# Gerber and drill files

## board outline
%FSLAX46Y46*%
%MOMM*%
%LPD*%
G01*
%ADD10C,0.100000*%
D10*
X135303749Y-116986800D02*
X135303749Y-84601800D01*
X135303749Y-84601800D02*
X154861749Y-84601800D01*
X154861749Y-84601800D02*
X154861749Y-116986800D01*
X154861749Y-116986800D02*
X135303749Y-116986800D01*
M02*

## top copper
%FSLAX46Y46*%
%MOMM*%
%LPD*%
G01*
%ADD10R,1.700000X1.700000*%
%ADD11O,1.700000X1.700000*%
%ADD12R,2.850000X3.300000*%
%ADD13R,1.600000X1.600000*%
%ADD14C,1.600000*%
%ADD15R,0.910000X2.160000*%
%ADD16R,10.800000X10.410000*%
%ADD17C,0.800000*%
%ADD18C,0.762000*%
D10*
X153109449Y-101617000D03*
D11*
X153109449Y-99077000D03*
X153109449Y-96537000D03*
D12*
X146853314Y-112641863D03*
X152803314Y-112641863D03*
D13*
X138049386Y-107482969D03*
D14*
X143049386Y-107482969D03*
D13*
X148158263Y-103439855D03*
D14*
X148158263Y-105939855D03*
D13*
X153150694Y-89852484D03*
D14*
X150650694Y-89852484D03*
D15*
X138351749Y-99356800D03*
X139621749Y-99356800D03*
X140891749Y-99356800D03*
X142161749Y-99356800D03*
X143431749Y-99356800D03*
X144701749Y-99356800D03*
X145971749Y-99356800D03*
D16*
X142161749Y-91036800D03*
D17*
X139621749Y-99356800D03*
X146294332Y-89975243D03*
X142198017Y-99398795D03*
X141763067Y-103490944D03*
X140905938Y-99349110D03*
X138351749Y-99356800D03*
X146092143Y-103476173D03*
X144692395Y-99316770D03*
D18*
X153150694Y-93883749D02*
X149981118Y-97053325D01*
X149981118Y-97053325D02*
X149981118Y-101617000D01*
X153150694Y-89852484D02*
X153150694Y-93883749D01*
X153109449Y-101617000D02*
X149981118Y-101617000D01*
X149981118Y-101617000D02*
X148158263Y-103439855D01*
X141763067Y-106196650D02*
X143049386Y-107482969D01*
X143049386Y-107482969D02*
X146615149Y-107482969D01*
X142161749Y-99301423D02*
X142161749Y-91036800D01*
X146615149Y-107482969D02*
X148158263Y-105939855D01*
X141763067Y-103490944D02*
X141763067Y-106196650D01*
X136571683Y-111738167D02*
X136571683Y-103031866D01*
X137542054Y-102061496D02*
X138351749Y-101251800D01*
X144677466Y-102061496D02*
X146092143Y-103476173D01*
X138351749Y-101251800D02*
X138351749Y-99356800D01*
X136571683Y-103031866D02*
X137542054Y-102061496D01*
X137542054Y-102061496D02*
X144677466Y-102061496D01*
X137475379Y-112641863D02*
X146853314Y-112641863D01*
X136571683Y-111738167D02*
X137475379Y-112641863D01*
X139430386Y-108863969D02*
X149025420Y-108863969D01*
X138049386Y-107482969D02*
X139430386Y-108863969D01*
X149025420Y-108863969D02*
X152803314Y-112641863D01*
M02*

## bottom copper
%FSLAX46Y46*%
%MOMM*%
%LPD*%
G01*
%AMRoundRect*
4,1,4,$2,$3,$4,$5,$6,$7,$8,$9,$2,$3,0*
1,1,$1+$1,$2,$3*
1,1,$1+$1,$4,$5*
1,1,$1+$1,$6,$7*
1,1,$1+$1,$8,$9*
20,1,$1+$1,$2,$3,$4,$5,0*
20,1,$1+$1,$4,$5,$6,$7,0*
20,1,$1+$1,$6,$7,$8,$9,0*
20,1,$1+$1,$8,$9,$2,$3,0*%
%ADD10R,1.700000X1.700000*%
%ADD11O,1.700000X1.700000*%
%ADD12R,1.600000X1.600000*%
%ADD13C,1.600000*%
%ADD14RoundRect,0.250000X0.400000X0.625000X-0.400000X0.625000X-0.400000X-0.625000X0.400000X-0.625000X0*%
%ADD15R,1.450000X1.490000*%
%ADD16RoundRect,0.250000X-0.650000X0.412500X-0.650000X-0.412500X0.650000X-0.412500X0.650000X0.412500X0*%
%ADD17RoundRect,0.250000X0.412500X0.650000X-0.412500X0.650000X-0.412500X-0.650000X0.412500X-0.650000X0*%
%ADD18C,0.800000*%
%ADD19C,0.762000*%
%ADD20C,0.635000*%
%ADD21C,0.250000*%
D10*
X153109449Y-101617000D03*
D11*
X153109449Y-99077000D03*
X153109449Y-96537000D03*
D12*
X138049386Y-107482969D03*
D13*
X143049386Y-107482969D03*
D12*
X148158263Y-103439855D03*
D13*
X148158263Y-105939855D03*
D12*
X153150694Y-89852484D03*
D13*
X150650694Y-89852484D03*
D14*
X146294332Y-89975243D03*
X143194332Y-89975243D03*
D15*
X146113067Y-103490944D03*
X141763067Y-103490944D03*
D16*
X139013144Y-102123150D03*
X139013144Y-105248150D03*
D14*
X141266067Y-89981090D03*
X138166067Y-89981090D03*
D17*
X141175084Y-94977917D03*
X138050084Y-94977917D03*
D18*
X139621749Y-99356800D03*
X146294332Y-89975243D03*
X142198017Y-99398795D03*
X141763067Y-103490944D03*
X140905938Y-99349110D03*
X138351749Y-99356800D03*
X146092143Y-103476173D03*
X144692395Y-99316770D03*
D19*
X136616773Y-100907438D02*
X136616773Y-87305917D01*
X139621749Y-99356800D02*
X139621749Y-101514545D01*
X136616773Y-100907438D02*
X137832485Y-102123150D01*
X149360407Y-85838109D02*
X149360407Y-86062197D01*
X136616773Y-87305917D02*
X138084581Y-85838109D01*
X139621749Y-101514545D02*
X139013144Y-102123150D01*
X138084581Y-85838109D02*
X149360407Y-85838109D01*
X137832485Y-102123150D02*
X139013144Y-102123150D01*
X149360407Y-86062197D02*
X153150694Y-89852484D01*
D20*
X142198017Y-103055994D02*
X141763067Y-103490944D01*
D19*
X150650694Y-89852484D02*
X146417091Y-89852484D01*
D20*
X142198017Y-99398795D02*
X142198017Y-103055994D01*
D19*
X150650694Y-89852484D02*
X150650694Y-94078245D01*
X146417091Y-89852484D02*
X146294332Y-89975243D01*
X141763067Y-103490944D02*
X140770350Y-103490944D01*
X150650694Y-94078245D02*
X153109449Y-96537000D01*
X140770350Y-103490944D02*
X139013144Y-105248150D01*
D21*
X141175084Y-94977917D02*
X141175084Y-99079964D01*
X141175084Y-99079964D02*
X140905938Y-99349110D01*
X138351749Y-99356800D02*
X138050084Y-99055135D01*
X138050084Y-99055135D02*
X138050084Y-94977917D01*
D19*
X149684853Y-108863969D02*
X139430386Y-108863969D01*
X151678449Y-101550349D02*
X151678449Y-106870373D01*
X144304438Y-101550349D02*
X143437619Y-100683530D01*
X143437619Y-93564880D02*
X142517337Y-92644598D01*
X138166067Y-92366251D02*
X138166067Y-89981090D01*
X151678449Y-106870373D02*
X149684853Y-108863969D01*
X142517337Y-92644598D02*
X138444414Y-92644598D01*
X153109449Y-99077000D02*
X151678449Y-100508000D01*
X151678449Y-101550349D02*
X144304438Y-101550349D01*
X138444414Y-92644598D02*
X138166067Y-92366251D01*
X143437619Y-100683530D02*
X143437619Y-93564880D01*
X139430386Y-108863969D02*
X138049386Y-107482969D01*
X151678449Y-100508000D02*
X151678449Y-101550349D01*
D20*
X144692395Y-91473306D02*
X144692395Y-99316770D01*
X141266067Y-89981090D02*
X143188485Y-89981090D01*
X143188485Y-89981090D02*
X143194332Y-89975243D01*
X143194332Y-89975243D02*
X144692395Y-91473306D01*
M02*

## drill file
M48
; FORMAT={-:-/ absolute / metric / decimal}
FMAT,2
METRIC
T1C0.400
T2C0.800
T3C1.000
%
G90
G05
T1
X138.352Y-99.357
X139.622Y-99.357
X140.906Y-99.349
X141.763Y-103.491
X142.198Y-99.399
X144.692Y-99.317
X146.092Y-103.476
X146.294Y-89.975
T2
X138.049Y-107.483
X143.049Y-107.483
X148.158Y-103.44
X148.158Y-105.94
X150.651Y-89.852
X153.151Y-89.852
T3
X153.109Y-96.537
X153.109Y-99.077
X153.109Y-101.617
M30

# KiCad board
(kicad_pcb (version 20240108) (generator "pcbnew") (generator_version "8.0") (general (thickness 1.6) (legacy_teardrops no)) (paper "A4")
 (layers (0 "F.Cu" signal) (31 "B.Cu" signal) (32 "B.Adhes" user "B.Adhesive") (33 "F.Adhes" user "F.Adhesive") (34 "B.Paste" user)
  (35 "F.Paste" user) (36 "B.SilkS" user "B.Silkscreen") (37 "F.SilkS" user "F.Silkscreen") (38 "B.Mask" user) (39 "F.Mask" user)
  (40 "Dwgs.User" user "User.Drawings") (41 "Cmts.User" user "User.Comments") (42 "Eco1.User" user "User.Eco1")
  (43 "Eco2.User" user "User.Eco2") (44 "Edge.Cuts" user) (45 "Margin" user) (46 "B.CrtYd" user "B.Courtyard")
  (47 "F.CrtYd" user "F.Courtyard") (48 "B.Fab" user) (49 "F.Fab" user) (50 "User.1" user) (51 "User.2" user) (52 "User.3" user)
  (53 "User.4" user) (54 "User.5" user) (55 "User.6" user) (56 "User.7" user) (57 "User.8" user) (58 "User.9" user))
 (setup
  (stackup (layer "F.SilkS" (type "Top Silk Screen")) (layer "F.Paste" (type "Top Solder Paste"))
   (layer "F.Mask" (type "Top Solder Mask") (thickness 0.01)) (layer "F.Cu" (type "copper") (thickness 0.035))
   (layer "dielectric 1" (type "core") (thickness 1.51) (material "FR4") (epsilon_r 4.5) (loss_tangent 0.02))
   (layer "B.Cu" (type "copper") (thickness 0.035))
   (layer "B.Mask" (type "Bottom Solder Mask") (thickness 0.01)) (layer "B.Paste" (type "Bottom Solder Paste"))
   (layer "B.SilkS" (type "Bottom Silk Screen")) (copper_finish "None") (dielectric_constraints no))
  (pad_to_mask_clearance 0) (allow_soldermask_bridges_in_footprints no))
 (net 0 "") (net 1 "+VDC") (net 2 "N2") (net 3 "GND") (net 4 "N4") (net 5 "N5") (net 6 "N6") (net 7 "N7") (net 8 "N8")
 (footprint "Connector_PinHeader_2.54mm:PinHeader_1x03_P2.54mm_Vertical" (layer "F.Cu") (at 153.109449 101.617 180)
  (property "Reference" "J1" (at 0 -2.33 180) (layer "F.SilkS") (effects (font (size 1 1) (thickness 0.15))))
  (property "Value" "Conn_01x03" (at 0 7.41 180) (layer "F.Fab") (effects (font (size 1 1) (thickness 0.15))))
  (pad "1" thru_hole rect (at 0 0 180) (size 1.7 1.7) (drill 1) (layers "*.Cu" "*.Mask") (remove_unused_layers no) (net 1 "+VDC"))
  (pad "2" thru_hole oval (at 0 2.54 180) (size 1.7 1.7) (drill 1) (layers "*.Cu" "*.Mask") (remove_unused_layers no) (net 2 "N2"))
  (pad "3" thru_hole oval (at 0 5.08 180) (size 1.7 1.7) (drill 1) (layers "*.Cu" "*.Mask") (remove_unused_layers no) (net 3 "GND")))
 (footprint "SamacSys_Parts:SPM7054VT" (layer "F.Cu") (at 149.828314 112.641863)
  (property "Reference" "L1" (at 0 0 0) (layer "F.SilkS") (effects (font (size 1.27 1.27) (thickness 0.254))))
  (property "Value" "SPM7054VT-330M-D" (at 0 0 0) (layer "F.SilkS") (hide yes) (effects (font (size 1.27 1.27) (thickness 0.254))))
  (pad "1" smd rect (at -2.975 0) (size 2.85 3.3) (layers "F.Cu" "F.Paste" "F.Mask") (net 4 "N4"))
  (pad "2" smd rect (at 2.975 0) (size 2.85 3.3) (layers "F.Cu" "F.Paste" "F.Mask") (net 2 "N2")))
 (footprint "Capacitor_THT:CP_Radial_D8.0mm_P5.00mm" (layer "F.Cu") (at 138.049386 107.482969)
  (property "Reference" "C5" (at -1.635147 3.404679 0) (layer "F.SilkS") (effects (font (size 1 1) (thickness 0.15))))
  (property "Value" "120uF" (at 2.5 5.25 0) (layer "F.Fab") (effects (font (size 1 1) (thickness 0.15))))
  (pad "1" thru_hole rect (at 0 0) (size 1.6 1.6) (drill 0.8) (layers "*.Cu" "*.Mask") (remove_unused_layers no) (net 2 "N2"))
  (pad "2" thru_hole circle (at 5 0) (size 1.6 1.6) (drill 0.8) (layers "*.Cu" "*.Mask") (remove_unused_layers no) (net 3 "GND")))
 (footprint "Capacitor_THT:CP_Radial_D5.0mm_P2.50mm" (layer "F.Cu") (at 148.158263 103.439855 -90)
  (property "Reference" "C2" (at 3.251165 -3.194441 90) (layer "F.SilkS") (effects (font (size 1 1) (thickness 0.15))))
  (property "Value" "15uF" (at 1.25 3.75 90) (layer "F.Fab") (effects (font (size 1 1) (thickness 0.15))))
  (pad "1" thru_hole rect (at 0 0 270) (size 1.6 1.6) (drill 0.8) (layers "*.Cu" "*.Mask") (remove_unused_layers no) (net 1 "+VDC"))
  (pad "2" thru_hole circle (at 2.5 0 270) (size 1.6 1.6) (drill 0.8) (layers "*.Cu" "*.Mask") (remove_unused_layers no) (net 3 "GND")))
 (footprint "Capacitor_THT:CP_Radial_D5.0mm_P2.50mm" (layer "F.Cu") (at 153.150694 89.852484 180)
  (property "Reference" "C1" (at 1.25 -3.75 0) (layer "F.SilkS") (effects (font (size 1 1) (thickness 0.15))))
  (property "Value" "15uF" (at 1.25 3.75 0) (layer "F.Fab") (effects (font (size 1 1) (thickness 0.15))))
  (pad "1" thru_hole rect (at 0 0 180) (size 1.6 1.6) (drill 0.8) (layers "*.Cu" "*.Mask") (remove_unused_layers no) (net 1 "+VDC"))
  (pad "2" thru_hole circle (at 2.5 0 180) (size 1.6 1.6) (drill 0.8) (layers "*.Cu" "*.Mask") (remove_unused_layers no) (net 3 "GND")))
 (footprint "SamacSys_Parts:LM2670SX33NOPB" (layer "F.Cu") (at 142.161749 91.5868 -90)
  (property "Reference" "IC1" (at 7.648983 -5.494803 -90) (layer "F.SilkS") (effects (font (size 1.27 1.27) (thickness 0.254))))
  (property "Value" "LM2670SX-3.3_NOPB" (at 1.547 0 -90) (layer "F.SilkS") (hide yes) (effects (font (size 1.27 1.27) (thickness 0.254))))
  (pad "1" smd rect (at 7.77 3.81) (size 0.91 2.16) (layers "F.Cu" "F.Paste" "F.Mask") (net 4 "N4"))
  (pad "2" smd rect (at 7.77 2.54) (size 0.91 2.16) (layers "F.Cu" "F.Paste" "F.Mask") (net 1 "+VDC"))
  (pad "3" smd rect (at 7.77 1.27) (size 0.91 2.16) (layers "F.Cu" "F.Paste" "F.Mask") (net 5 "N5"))
  (pad "4" smd rect (at 7.77 0) (size 0.91 2.16) (layers "F.Cu" "F.Paste" "F.Mask") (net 3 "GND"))
  (pad "5" smd rect (at 7.77 -1.27) (size 0.91 2.16) (layers "F.Cu" "F.Paste" "F.Mask") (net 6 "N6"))
  (pad "6" smd rect (at 7.77 -2.54) (size 0.91 2.16) (layers "F.Cu" "F.Paste" "F.Mask") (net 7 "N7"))
  (pad "7" smd rect (at 7.77 -3.81) (size 0.91 2.16) (layers "F.Cu" "F.Paste" "F.Mask") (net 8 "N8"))
  (pad "8" smd rect (at -0.55 0 270) (size 10.41 10.8) (layers "F.Cu" "F.Paste" "F.Mask") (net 3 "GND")))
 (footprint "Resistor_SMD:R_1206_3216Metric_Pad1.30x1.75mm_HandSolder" (layer "B.Cu") (at 144.744332 89.975243 180)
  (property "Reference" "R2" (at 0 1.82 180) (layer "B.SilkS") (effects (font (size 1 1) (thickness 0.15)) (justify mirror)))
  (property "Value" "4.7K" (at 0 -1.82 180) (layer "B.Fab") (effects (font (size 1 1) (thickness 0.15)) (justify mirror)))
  (pad "1" smd roundrect (at -1.55 0 180) (size 1.3 1.75) (layers "B.Cu" "B.Paste" "B.Mask") (roundrect_rratio 0.192308) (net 3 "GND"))
  (pad "2" smd roundrect (at 1.55 0 180) (size 1.3 1.75) (layers "B.Cu" "B.Paste" "B.Mask") (roundrect_rratio 0.192308) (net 7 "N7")))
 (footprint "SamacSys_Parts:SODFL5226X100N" (layer "B.Cu") (at 143.938067 103.490944 180)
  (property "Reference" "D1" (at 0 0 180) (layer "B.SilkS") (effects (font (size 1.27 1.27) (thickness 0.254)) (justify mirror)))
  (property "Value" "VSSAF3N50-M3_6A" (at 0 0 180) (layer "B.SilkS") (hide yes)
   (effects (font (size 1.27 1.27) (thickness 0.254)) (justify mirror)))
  (pad "1" smd rect (at -2.175 0 180) (size 1.45 1.49) (layers "B.Cu" "B.Paste" "B.Mask") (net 4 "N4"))
  (pad "2" smd rect (at 2.175 0 180) (size 1.45 1.49) (layers "B.Cu" "B.Paste" "B.Mask") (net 3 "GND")))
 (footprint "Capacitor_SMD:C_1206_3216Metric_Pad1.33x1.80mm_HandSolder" (layer "B.Cu") (at 139.013144 103.68565 -90)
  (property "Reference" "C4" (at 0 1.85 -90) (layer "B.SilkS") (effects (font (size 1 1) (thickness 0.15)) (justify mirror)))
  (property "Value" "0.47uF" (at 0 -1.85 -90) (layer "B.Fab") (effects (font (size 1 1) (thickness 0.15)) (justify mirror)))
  (pad "1" smd roundrect (at -1.5625 0 270) (size 1.325 1.8) (layers "B.Cu" "B.Paste" "B.Mask") (roundrect_rratio 0.188679) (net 1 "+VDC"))
  (pad "2" smd roundrect (at 1.5625 0 270) (size 1.325 1.8) (layers "B.Cu" "B.Paste" "B.Mask") (roundrect_rratio 0.188679) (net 3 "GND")))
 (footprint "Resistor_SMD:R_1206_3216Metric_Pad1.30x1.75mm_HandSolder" (layer "B.Cu") (at 139.716067 89.98109 180)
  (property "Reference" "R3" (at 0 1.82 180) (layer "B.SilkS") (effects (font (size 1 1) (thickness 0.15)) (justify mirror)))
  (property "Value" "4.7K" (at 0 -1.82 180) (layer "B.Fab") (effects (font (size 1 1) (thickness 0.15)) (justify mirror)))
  (pad "1" smd roundrect (at -1.55 0 180) (size 1.3 1.75) (layers "B.Cu" "B.Paste" "B.Mask") (roundrect_rratio 0.192308) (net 7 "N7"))
  (pad "2" smd roundrect (at 1.55 0 180) (size 1.3 1.75) (layers "B.Cu" "B.Paste" "B.Mask") (roundrect_rratio 0.192308) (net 2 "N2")))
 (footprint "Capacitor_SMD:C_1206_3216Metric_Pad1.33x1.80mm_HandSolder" (layer "B.Cu") (at 139.612584 94.977917 180)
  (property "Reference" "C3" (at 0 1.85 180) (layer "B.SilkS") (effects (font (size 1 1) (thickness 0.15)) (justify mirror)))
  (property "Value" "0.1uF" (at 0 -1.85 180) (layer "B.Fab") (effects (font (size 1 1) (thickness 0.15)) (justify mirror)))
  (pad "1" smd roundrect (at -1.5625 0 180) (size 1.325 1.8) (layers "B.Cu" "B.Paste" "B.Mask") (roundrect_rratio 0.188679) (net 5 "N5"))
  (pad "2" smd roundrect (at 1.5625 0 180) (size 1.325 1.8) (layers "B.Cu" "B.Paste" "B.Mask") (roundrect_rratio 0.188679) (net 4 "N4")))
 (gr_line (start 135.303749 116.9868) (end 135.303749 84.6018) (stroke (width 0.1) (type solid)) (layer "Edge.Cuts"))
 (gr_line (start 135.303749 84.6018) (end 154.861749 84.6018) (stroke (width 0.1) (type solid)) (layer "Edge.Cuts"))
 (gr_line (start 154.861749 84.6018) (end 154.861749 116.9868) (stroke (width 0.1) (type default)) (layer "Edge.Cuts"))
 (gr_line (start 154.861749 116.9868) (end 135.303749 116.9868) (stroke (width 0.1) (type default)) (layer "Edge.Cuts"))
 (segment (start 153.150694 93.883749) (end 149.981118 97.053325) (width 0.762) (layer "F.Cu") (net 1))
 (segment (start 149.981118 97.053325) (end 149.981118 101.617) (width 0.762) (layer "F.Cu") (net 1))
 (segment (start 153.150694 89.852484) (end 153.150694 93.883749) (width 0.762) (layer "F.Cu") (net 1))
 (segment (start 153.109449 101.617) (end 149.981118 101.617) (width 0.762) (layer "F.Cu") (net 1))
 (segment (start 149.981118 101.617) (end 148.158263 103.439855) (width 0.762) (layer "F.Cu") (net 1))
 (via (at 139.621749 99.3568) (size 0.8) (drill 0.4) (layers "F.Cu" "B.Cu") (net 1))
 (segment (start 136.616773 100.907438) (end 136.616773 87.305917) (width 0.762) (layer "B.Cu") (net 1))
 (segment (start 139.621749 99.3568) (end 139.621749 101.514545) (width 0.762) (layer "B.Cu") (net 1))
 (segment (start 136.616773 100.907438) (end 137.832485 102.12315) (width 0.762) (layer "B.Cu") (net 1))
 (segment (start 149.360407 85.838109) (end 149.360407 86.062197) (width 0.762) (layer "B.Cu") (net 1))
 (segment (start 136.616773 87.305917) (end 138.084581 85.838109) (width 0.762) (layer "B.Cu") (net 1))
 (segment (start 139.621749 101.514545) (end 139.013144 102.12315) (width 0.762) (layer "B.Cu") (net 1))
 (segment (start 138.084581 85.838109) (end 149.360407 85.838109) (width 0.762) (layer "B.Cu") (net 1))
 (segment (start 137.832485 102.12315) (end 139.013144 102.12315) (width 0.762) (layer "B.Cu") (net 1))
 (segment (start 149.360407 86.062197) (end 153.150694 89.852484) (width 0.762) (layer "B.Cu") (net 1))
 (segment (start 141.763067 106.19665) (end 143.049386 107.482969) (width 0.762) (layer "F.Cu") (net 3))
 (segment (start 143.049386 107.482969) (end 146.615149 107.482969) (width 0.762) (layer "F.Cu") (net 3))
 (segment (start 142.161749 99.301423) (end 142.161749 91.0368) (width 0.762) (layer "F.Cu") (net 3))
 (segment (start 146.615149 107.482969) (end 148.158263 105.939855) (width 0.762) (layer "F.Cu") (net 3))
 (segment (start 141.763067 103.490944) (end 141.763067 106.19665) (width 0.762) (layer "F.Cu") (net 3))
 (via (at 146.294332 89.975243) (size 0.8) (drill 0.4) (layers "F.Cu" "B.Cu") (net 3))
 (via (at 142.198017 99.398795) (size 0.8) (drill 0.4) (layers "F.Cu" "B.Cu") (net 3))
 (via (at 141.763067 103.490944) (size 0.8) (drill 0.4) (layers "F.Cu" "B.Cu") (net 3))
 (segment (start 142.198017 103.055994) (end 141.763067 103.490944) (width 0.635) (layer "B.Cu") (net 3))
 (segment (start 150.650694 89.852484) (end 146.417091 89.852484) (width 0.762) (layer "B.Cu") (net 3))
 (segment (start 142.198017 99.398795) (end 142.198017 103.055994) (width 0.635) (layer "B.Cu") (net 3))
 (segment (start 150.650694 89.852484) (end 150.650694 94.078245) (width 0.762) (layer "B.Cu") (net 3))
 (segment (start 146.417091 89.852484) (end 146.294332 89.975243) (width 0.762) (layer "B.Cu") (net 3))
 (segment (start 141.763067 103.490944) (end 140.77035 103.490944) (width 0.762) (layer "B.Cu") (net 3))
 (segment (start 150.650694 94.078245) (end 153.109449 96.537) (width 0.762) (layer "B.Cu") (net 3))
 (segment (start 140.77035 103.490944) (end 139.013144 105.24815) (width 0.762) (layer "B.Cu") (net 3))
 (via (at 140.905938 99.34911) (size 0.8) (drill 0.4) (layers "F.Cu" "B.Cu") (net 5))
 (segment (start 141.175084 94.977917) (end 141.175084 99.079964) (width 0.25) (layer "B.Cu") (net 5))
 (segment (start 141.175084 99.079964) (end 140.905938 99.34911) (width 0.25) (layer "B.Cu") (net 5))
 (segment (start 136.571683 111.738167) (end 136.571683 103.031866) (width 0.762) (layer "F.Cu") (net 4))
 (segment (start 137.542054 102.061496) (end 138.351749 101.2518) (width 0.762) (layer "F.Cu") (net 4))
 (segment (start 144.677466 102.061496) (end 146.092143 103.476173) (width 0.762) (layer "F.Cu") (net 4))
 (segment (start 138.351749 101.2518) (end 138.351749 99.3568) (width 0.762) (layer "F.Cu") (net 4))
 (segment (start 136.571683 103.031866) (end 137.542054 102.061496) (width 0.762) (layer "F.Cu") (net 4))
 (segment (start 137.542054 102.061496) (end 144.677466 102.061496) (width 0.762) (layer "F.Cu") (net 4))
 (segment (start 137.475379 112.641863) (end 146.853314 112.641863) (width 0.762) (layer "F.Cu") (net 4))
 (segment (start 136.571683 111.738167) (end 137.475379 112.641863) (width 0.762) (layer "F.Cu") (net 4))
 (via (at 138.351749 99.3568) (size 0.8) (drill 0.4) (layers "F.Cu" "B.Cu") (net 4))
 (via (at 146.092143 103.476173) (size 0.8) (drill 0.4) (layers "F.Cu" "B.Cu") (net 4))
 (segment (start 138.351749 99.3568) (end 138.050084 99.055135) (width 0.25) (layer "B.Cu") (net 4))
 (segment (start 138.050084 99.055135) (end 138.050084 94.977917) (width 0.25) (layer "B.Cu") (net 4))
 (segment (start 139.430386 108.863969) (end 149.02542 108.863969) (width 0.762) (layer "F.Cu") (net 2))
 (segment (start 138.049386 107.482969) (end 139.430386 108.863969) (width 0.762) (layer "F.Cu") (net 2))
 (segment (start 149.02542 108.863969) (end 152.803314 112.641863) (width 0.762) (layer "F.Cu") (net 2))
 (segment (start 149.684853 108.863969) (end 139.430386 108.863969) (width 0.762) (layer "B.Cu") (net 2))
 (segment (start 151.678449 101.550349) (end 151.678449 106.870373) (width 0.762) (layer "B.Cu") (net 2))
 (segment (start 144.304438 101.550349) (end 143.437619 100.68353) (width 0.762) (layer "B.Cu") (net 2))
 (segment (start 143.437619 93.56488) (end 142.517337 92.644598) (width 0.762) (layer "B.Cu") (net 2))
 (segment (start 138.166067 92.366251) (end 138.166067 89.98109) (width 0.762) (layer "B.Cu") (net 2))
 (segment (start 151.678449 106.870373) (end 149.684853 108.863969) (width 0.762) (layer "B.Cu") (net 2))
 (segment (start 142.517337 92.644598) (end 138.444414 92.644598) (width 0.762) (layer "B.Cu") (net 2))
 (segment (start 153.109449 99.077) (end 151.678449 100.508) (width 0.762) (layer "B.Cu") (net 2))
 (segment (start 151.678449 101.550349) (end 144.304438 101.550349) (width 0.762) (layer "B.Cu") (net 2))
 (segment (start 138.444414 92.644598) (end 138.166067 92.366251) (width 0.762) (layer "B.Cu") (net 2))
 (segment (start 143.437619 100.68353) (end 143.437619 93.56488) (width 0.762) (layer "B.Cu") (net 2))
 (segment (start 139.430386 108.863969) (end 138.049386 107.482969) (width 0.762) (layer "B.Cu") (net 2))
 (segment (start 151.678449 100.508) (end 151.678449 101.550349) (width 0.762) (layer "B.Cu") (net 2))
 (via (at 144.692395 99.31677) (size 0.8) (drill 0.4) (layers "F.Cu" "B.Cu") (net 7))
 (segment (start 144.692395 91.473306) (end 144.692395 99.31677) (width 0.635) (layer "B.Cu") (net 7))
 (segment (start 141.266067 89.98109) (end 143.188485 89.98109) (width 0.635) (layer "B.Cu") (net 7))
 (segment (start 143.188485 89.98109) (end 143.194332 89.975243) (width 0.635) (layer "B.Cu") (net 7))
 (segment (start 143.194332 89.975243) (end 144.692395 91.473306) (width 0.635) (layer "B.Cu") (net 7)))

